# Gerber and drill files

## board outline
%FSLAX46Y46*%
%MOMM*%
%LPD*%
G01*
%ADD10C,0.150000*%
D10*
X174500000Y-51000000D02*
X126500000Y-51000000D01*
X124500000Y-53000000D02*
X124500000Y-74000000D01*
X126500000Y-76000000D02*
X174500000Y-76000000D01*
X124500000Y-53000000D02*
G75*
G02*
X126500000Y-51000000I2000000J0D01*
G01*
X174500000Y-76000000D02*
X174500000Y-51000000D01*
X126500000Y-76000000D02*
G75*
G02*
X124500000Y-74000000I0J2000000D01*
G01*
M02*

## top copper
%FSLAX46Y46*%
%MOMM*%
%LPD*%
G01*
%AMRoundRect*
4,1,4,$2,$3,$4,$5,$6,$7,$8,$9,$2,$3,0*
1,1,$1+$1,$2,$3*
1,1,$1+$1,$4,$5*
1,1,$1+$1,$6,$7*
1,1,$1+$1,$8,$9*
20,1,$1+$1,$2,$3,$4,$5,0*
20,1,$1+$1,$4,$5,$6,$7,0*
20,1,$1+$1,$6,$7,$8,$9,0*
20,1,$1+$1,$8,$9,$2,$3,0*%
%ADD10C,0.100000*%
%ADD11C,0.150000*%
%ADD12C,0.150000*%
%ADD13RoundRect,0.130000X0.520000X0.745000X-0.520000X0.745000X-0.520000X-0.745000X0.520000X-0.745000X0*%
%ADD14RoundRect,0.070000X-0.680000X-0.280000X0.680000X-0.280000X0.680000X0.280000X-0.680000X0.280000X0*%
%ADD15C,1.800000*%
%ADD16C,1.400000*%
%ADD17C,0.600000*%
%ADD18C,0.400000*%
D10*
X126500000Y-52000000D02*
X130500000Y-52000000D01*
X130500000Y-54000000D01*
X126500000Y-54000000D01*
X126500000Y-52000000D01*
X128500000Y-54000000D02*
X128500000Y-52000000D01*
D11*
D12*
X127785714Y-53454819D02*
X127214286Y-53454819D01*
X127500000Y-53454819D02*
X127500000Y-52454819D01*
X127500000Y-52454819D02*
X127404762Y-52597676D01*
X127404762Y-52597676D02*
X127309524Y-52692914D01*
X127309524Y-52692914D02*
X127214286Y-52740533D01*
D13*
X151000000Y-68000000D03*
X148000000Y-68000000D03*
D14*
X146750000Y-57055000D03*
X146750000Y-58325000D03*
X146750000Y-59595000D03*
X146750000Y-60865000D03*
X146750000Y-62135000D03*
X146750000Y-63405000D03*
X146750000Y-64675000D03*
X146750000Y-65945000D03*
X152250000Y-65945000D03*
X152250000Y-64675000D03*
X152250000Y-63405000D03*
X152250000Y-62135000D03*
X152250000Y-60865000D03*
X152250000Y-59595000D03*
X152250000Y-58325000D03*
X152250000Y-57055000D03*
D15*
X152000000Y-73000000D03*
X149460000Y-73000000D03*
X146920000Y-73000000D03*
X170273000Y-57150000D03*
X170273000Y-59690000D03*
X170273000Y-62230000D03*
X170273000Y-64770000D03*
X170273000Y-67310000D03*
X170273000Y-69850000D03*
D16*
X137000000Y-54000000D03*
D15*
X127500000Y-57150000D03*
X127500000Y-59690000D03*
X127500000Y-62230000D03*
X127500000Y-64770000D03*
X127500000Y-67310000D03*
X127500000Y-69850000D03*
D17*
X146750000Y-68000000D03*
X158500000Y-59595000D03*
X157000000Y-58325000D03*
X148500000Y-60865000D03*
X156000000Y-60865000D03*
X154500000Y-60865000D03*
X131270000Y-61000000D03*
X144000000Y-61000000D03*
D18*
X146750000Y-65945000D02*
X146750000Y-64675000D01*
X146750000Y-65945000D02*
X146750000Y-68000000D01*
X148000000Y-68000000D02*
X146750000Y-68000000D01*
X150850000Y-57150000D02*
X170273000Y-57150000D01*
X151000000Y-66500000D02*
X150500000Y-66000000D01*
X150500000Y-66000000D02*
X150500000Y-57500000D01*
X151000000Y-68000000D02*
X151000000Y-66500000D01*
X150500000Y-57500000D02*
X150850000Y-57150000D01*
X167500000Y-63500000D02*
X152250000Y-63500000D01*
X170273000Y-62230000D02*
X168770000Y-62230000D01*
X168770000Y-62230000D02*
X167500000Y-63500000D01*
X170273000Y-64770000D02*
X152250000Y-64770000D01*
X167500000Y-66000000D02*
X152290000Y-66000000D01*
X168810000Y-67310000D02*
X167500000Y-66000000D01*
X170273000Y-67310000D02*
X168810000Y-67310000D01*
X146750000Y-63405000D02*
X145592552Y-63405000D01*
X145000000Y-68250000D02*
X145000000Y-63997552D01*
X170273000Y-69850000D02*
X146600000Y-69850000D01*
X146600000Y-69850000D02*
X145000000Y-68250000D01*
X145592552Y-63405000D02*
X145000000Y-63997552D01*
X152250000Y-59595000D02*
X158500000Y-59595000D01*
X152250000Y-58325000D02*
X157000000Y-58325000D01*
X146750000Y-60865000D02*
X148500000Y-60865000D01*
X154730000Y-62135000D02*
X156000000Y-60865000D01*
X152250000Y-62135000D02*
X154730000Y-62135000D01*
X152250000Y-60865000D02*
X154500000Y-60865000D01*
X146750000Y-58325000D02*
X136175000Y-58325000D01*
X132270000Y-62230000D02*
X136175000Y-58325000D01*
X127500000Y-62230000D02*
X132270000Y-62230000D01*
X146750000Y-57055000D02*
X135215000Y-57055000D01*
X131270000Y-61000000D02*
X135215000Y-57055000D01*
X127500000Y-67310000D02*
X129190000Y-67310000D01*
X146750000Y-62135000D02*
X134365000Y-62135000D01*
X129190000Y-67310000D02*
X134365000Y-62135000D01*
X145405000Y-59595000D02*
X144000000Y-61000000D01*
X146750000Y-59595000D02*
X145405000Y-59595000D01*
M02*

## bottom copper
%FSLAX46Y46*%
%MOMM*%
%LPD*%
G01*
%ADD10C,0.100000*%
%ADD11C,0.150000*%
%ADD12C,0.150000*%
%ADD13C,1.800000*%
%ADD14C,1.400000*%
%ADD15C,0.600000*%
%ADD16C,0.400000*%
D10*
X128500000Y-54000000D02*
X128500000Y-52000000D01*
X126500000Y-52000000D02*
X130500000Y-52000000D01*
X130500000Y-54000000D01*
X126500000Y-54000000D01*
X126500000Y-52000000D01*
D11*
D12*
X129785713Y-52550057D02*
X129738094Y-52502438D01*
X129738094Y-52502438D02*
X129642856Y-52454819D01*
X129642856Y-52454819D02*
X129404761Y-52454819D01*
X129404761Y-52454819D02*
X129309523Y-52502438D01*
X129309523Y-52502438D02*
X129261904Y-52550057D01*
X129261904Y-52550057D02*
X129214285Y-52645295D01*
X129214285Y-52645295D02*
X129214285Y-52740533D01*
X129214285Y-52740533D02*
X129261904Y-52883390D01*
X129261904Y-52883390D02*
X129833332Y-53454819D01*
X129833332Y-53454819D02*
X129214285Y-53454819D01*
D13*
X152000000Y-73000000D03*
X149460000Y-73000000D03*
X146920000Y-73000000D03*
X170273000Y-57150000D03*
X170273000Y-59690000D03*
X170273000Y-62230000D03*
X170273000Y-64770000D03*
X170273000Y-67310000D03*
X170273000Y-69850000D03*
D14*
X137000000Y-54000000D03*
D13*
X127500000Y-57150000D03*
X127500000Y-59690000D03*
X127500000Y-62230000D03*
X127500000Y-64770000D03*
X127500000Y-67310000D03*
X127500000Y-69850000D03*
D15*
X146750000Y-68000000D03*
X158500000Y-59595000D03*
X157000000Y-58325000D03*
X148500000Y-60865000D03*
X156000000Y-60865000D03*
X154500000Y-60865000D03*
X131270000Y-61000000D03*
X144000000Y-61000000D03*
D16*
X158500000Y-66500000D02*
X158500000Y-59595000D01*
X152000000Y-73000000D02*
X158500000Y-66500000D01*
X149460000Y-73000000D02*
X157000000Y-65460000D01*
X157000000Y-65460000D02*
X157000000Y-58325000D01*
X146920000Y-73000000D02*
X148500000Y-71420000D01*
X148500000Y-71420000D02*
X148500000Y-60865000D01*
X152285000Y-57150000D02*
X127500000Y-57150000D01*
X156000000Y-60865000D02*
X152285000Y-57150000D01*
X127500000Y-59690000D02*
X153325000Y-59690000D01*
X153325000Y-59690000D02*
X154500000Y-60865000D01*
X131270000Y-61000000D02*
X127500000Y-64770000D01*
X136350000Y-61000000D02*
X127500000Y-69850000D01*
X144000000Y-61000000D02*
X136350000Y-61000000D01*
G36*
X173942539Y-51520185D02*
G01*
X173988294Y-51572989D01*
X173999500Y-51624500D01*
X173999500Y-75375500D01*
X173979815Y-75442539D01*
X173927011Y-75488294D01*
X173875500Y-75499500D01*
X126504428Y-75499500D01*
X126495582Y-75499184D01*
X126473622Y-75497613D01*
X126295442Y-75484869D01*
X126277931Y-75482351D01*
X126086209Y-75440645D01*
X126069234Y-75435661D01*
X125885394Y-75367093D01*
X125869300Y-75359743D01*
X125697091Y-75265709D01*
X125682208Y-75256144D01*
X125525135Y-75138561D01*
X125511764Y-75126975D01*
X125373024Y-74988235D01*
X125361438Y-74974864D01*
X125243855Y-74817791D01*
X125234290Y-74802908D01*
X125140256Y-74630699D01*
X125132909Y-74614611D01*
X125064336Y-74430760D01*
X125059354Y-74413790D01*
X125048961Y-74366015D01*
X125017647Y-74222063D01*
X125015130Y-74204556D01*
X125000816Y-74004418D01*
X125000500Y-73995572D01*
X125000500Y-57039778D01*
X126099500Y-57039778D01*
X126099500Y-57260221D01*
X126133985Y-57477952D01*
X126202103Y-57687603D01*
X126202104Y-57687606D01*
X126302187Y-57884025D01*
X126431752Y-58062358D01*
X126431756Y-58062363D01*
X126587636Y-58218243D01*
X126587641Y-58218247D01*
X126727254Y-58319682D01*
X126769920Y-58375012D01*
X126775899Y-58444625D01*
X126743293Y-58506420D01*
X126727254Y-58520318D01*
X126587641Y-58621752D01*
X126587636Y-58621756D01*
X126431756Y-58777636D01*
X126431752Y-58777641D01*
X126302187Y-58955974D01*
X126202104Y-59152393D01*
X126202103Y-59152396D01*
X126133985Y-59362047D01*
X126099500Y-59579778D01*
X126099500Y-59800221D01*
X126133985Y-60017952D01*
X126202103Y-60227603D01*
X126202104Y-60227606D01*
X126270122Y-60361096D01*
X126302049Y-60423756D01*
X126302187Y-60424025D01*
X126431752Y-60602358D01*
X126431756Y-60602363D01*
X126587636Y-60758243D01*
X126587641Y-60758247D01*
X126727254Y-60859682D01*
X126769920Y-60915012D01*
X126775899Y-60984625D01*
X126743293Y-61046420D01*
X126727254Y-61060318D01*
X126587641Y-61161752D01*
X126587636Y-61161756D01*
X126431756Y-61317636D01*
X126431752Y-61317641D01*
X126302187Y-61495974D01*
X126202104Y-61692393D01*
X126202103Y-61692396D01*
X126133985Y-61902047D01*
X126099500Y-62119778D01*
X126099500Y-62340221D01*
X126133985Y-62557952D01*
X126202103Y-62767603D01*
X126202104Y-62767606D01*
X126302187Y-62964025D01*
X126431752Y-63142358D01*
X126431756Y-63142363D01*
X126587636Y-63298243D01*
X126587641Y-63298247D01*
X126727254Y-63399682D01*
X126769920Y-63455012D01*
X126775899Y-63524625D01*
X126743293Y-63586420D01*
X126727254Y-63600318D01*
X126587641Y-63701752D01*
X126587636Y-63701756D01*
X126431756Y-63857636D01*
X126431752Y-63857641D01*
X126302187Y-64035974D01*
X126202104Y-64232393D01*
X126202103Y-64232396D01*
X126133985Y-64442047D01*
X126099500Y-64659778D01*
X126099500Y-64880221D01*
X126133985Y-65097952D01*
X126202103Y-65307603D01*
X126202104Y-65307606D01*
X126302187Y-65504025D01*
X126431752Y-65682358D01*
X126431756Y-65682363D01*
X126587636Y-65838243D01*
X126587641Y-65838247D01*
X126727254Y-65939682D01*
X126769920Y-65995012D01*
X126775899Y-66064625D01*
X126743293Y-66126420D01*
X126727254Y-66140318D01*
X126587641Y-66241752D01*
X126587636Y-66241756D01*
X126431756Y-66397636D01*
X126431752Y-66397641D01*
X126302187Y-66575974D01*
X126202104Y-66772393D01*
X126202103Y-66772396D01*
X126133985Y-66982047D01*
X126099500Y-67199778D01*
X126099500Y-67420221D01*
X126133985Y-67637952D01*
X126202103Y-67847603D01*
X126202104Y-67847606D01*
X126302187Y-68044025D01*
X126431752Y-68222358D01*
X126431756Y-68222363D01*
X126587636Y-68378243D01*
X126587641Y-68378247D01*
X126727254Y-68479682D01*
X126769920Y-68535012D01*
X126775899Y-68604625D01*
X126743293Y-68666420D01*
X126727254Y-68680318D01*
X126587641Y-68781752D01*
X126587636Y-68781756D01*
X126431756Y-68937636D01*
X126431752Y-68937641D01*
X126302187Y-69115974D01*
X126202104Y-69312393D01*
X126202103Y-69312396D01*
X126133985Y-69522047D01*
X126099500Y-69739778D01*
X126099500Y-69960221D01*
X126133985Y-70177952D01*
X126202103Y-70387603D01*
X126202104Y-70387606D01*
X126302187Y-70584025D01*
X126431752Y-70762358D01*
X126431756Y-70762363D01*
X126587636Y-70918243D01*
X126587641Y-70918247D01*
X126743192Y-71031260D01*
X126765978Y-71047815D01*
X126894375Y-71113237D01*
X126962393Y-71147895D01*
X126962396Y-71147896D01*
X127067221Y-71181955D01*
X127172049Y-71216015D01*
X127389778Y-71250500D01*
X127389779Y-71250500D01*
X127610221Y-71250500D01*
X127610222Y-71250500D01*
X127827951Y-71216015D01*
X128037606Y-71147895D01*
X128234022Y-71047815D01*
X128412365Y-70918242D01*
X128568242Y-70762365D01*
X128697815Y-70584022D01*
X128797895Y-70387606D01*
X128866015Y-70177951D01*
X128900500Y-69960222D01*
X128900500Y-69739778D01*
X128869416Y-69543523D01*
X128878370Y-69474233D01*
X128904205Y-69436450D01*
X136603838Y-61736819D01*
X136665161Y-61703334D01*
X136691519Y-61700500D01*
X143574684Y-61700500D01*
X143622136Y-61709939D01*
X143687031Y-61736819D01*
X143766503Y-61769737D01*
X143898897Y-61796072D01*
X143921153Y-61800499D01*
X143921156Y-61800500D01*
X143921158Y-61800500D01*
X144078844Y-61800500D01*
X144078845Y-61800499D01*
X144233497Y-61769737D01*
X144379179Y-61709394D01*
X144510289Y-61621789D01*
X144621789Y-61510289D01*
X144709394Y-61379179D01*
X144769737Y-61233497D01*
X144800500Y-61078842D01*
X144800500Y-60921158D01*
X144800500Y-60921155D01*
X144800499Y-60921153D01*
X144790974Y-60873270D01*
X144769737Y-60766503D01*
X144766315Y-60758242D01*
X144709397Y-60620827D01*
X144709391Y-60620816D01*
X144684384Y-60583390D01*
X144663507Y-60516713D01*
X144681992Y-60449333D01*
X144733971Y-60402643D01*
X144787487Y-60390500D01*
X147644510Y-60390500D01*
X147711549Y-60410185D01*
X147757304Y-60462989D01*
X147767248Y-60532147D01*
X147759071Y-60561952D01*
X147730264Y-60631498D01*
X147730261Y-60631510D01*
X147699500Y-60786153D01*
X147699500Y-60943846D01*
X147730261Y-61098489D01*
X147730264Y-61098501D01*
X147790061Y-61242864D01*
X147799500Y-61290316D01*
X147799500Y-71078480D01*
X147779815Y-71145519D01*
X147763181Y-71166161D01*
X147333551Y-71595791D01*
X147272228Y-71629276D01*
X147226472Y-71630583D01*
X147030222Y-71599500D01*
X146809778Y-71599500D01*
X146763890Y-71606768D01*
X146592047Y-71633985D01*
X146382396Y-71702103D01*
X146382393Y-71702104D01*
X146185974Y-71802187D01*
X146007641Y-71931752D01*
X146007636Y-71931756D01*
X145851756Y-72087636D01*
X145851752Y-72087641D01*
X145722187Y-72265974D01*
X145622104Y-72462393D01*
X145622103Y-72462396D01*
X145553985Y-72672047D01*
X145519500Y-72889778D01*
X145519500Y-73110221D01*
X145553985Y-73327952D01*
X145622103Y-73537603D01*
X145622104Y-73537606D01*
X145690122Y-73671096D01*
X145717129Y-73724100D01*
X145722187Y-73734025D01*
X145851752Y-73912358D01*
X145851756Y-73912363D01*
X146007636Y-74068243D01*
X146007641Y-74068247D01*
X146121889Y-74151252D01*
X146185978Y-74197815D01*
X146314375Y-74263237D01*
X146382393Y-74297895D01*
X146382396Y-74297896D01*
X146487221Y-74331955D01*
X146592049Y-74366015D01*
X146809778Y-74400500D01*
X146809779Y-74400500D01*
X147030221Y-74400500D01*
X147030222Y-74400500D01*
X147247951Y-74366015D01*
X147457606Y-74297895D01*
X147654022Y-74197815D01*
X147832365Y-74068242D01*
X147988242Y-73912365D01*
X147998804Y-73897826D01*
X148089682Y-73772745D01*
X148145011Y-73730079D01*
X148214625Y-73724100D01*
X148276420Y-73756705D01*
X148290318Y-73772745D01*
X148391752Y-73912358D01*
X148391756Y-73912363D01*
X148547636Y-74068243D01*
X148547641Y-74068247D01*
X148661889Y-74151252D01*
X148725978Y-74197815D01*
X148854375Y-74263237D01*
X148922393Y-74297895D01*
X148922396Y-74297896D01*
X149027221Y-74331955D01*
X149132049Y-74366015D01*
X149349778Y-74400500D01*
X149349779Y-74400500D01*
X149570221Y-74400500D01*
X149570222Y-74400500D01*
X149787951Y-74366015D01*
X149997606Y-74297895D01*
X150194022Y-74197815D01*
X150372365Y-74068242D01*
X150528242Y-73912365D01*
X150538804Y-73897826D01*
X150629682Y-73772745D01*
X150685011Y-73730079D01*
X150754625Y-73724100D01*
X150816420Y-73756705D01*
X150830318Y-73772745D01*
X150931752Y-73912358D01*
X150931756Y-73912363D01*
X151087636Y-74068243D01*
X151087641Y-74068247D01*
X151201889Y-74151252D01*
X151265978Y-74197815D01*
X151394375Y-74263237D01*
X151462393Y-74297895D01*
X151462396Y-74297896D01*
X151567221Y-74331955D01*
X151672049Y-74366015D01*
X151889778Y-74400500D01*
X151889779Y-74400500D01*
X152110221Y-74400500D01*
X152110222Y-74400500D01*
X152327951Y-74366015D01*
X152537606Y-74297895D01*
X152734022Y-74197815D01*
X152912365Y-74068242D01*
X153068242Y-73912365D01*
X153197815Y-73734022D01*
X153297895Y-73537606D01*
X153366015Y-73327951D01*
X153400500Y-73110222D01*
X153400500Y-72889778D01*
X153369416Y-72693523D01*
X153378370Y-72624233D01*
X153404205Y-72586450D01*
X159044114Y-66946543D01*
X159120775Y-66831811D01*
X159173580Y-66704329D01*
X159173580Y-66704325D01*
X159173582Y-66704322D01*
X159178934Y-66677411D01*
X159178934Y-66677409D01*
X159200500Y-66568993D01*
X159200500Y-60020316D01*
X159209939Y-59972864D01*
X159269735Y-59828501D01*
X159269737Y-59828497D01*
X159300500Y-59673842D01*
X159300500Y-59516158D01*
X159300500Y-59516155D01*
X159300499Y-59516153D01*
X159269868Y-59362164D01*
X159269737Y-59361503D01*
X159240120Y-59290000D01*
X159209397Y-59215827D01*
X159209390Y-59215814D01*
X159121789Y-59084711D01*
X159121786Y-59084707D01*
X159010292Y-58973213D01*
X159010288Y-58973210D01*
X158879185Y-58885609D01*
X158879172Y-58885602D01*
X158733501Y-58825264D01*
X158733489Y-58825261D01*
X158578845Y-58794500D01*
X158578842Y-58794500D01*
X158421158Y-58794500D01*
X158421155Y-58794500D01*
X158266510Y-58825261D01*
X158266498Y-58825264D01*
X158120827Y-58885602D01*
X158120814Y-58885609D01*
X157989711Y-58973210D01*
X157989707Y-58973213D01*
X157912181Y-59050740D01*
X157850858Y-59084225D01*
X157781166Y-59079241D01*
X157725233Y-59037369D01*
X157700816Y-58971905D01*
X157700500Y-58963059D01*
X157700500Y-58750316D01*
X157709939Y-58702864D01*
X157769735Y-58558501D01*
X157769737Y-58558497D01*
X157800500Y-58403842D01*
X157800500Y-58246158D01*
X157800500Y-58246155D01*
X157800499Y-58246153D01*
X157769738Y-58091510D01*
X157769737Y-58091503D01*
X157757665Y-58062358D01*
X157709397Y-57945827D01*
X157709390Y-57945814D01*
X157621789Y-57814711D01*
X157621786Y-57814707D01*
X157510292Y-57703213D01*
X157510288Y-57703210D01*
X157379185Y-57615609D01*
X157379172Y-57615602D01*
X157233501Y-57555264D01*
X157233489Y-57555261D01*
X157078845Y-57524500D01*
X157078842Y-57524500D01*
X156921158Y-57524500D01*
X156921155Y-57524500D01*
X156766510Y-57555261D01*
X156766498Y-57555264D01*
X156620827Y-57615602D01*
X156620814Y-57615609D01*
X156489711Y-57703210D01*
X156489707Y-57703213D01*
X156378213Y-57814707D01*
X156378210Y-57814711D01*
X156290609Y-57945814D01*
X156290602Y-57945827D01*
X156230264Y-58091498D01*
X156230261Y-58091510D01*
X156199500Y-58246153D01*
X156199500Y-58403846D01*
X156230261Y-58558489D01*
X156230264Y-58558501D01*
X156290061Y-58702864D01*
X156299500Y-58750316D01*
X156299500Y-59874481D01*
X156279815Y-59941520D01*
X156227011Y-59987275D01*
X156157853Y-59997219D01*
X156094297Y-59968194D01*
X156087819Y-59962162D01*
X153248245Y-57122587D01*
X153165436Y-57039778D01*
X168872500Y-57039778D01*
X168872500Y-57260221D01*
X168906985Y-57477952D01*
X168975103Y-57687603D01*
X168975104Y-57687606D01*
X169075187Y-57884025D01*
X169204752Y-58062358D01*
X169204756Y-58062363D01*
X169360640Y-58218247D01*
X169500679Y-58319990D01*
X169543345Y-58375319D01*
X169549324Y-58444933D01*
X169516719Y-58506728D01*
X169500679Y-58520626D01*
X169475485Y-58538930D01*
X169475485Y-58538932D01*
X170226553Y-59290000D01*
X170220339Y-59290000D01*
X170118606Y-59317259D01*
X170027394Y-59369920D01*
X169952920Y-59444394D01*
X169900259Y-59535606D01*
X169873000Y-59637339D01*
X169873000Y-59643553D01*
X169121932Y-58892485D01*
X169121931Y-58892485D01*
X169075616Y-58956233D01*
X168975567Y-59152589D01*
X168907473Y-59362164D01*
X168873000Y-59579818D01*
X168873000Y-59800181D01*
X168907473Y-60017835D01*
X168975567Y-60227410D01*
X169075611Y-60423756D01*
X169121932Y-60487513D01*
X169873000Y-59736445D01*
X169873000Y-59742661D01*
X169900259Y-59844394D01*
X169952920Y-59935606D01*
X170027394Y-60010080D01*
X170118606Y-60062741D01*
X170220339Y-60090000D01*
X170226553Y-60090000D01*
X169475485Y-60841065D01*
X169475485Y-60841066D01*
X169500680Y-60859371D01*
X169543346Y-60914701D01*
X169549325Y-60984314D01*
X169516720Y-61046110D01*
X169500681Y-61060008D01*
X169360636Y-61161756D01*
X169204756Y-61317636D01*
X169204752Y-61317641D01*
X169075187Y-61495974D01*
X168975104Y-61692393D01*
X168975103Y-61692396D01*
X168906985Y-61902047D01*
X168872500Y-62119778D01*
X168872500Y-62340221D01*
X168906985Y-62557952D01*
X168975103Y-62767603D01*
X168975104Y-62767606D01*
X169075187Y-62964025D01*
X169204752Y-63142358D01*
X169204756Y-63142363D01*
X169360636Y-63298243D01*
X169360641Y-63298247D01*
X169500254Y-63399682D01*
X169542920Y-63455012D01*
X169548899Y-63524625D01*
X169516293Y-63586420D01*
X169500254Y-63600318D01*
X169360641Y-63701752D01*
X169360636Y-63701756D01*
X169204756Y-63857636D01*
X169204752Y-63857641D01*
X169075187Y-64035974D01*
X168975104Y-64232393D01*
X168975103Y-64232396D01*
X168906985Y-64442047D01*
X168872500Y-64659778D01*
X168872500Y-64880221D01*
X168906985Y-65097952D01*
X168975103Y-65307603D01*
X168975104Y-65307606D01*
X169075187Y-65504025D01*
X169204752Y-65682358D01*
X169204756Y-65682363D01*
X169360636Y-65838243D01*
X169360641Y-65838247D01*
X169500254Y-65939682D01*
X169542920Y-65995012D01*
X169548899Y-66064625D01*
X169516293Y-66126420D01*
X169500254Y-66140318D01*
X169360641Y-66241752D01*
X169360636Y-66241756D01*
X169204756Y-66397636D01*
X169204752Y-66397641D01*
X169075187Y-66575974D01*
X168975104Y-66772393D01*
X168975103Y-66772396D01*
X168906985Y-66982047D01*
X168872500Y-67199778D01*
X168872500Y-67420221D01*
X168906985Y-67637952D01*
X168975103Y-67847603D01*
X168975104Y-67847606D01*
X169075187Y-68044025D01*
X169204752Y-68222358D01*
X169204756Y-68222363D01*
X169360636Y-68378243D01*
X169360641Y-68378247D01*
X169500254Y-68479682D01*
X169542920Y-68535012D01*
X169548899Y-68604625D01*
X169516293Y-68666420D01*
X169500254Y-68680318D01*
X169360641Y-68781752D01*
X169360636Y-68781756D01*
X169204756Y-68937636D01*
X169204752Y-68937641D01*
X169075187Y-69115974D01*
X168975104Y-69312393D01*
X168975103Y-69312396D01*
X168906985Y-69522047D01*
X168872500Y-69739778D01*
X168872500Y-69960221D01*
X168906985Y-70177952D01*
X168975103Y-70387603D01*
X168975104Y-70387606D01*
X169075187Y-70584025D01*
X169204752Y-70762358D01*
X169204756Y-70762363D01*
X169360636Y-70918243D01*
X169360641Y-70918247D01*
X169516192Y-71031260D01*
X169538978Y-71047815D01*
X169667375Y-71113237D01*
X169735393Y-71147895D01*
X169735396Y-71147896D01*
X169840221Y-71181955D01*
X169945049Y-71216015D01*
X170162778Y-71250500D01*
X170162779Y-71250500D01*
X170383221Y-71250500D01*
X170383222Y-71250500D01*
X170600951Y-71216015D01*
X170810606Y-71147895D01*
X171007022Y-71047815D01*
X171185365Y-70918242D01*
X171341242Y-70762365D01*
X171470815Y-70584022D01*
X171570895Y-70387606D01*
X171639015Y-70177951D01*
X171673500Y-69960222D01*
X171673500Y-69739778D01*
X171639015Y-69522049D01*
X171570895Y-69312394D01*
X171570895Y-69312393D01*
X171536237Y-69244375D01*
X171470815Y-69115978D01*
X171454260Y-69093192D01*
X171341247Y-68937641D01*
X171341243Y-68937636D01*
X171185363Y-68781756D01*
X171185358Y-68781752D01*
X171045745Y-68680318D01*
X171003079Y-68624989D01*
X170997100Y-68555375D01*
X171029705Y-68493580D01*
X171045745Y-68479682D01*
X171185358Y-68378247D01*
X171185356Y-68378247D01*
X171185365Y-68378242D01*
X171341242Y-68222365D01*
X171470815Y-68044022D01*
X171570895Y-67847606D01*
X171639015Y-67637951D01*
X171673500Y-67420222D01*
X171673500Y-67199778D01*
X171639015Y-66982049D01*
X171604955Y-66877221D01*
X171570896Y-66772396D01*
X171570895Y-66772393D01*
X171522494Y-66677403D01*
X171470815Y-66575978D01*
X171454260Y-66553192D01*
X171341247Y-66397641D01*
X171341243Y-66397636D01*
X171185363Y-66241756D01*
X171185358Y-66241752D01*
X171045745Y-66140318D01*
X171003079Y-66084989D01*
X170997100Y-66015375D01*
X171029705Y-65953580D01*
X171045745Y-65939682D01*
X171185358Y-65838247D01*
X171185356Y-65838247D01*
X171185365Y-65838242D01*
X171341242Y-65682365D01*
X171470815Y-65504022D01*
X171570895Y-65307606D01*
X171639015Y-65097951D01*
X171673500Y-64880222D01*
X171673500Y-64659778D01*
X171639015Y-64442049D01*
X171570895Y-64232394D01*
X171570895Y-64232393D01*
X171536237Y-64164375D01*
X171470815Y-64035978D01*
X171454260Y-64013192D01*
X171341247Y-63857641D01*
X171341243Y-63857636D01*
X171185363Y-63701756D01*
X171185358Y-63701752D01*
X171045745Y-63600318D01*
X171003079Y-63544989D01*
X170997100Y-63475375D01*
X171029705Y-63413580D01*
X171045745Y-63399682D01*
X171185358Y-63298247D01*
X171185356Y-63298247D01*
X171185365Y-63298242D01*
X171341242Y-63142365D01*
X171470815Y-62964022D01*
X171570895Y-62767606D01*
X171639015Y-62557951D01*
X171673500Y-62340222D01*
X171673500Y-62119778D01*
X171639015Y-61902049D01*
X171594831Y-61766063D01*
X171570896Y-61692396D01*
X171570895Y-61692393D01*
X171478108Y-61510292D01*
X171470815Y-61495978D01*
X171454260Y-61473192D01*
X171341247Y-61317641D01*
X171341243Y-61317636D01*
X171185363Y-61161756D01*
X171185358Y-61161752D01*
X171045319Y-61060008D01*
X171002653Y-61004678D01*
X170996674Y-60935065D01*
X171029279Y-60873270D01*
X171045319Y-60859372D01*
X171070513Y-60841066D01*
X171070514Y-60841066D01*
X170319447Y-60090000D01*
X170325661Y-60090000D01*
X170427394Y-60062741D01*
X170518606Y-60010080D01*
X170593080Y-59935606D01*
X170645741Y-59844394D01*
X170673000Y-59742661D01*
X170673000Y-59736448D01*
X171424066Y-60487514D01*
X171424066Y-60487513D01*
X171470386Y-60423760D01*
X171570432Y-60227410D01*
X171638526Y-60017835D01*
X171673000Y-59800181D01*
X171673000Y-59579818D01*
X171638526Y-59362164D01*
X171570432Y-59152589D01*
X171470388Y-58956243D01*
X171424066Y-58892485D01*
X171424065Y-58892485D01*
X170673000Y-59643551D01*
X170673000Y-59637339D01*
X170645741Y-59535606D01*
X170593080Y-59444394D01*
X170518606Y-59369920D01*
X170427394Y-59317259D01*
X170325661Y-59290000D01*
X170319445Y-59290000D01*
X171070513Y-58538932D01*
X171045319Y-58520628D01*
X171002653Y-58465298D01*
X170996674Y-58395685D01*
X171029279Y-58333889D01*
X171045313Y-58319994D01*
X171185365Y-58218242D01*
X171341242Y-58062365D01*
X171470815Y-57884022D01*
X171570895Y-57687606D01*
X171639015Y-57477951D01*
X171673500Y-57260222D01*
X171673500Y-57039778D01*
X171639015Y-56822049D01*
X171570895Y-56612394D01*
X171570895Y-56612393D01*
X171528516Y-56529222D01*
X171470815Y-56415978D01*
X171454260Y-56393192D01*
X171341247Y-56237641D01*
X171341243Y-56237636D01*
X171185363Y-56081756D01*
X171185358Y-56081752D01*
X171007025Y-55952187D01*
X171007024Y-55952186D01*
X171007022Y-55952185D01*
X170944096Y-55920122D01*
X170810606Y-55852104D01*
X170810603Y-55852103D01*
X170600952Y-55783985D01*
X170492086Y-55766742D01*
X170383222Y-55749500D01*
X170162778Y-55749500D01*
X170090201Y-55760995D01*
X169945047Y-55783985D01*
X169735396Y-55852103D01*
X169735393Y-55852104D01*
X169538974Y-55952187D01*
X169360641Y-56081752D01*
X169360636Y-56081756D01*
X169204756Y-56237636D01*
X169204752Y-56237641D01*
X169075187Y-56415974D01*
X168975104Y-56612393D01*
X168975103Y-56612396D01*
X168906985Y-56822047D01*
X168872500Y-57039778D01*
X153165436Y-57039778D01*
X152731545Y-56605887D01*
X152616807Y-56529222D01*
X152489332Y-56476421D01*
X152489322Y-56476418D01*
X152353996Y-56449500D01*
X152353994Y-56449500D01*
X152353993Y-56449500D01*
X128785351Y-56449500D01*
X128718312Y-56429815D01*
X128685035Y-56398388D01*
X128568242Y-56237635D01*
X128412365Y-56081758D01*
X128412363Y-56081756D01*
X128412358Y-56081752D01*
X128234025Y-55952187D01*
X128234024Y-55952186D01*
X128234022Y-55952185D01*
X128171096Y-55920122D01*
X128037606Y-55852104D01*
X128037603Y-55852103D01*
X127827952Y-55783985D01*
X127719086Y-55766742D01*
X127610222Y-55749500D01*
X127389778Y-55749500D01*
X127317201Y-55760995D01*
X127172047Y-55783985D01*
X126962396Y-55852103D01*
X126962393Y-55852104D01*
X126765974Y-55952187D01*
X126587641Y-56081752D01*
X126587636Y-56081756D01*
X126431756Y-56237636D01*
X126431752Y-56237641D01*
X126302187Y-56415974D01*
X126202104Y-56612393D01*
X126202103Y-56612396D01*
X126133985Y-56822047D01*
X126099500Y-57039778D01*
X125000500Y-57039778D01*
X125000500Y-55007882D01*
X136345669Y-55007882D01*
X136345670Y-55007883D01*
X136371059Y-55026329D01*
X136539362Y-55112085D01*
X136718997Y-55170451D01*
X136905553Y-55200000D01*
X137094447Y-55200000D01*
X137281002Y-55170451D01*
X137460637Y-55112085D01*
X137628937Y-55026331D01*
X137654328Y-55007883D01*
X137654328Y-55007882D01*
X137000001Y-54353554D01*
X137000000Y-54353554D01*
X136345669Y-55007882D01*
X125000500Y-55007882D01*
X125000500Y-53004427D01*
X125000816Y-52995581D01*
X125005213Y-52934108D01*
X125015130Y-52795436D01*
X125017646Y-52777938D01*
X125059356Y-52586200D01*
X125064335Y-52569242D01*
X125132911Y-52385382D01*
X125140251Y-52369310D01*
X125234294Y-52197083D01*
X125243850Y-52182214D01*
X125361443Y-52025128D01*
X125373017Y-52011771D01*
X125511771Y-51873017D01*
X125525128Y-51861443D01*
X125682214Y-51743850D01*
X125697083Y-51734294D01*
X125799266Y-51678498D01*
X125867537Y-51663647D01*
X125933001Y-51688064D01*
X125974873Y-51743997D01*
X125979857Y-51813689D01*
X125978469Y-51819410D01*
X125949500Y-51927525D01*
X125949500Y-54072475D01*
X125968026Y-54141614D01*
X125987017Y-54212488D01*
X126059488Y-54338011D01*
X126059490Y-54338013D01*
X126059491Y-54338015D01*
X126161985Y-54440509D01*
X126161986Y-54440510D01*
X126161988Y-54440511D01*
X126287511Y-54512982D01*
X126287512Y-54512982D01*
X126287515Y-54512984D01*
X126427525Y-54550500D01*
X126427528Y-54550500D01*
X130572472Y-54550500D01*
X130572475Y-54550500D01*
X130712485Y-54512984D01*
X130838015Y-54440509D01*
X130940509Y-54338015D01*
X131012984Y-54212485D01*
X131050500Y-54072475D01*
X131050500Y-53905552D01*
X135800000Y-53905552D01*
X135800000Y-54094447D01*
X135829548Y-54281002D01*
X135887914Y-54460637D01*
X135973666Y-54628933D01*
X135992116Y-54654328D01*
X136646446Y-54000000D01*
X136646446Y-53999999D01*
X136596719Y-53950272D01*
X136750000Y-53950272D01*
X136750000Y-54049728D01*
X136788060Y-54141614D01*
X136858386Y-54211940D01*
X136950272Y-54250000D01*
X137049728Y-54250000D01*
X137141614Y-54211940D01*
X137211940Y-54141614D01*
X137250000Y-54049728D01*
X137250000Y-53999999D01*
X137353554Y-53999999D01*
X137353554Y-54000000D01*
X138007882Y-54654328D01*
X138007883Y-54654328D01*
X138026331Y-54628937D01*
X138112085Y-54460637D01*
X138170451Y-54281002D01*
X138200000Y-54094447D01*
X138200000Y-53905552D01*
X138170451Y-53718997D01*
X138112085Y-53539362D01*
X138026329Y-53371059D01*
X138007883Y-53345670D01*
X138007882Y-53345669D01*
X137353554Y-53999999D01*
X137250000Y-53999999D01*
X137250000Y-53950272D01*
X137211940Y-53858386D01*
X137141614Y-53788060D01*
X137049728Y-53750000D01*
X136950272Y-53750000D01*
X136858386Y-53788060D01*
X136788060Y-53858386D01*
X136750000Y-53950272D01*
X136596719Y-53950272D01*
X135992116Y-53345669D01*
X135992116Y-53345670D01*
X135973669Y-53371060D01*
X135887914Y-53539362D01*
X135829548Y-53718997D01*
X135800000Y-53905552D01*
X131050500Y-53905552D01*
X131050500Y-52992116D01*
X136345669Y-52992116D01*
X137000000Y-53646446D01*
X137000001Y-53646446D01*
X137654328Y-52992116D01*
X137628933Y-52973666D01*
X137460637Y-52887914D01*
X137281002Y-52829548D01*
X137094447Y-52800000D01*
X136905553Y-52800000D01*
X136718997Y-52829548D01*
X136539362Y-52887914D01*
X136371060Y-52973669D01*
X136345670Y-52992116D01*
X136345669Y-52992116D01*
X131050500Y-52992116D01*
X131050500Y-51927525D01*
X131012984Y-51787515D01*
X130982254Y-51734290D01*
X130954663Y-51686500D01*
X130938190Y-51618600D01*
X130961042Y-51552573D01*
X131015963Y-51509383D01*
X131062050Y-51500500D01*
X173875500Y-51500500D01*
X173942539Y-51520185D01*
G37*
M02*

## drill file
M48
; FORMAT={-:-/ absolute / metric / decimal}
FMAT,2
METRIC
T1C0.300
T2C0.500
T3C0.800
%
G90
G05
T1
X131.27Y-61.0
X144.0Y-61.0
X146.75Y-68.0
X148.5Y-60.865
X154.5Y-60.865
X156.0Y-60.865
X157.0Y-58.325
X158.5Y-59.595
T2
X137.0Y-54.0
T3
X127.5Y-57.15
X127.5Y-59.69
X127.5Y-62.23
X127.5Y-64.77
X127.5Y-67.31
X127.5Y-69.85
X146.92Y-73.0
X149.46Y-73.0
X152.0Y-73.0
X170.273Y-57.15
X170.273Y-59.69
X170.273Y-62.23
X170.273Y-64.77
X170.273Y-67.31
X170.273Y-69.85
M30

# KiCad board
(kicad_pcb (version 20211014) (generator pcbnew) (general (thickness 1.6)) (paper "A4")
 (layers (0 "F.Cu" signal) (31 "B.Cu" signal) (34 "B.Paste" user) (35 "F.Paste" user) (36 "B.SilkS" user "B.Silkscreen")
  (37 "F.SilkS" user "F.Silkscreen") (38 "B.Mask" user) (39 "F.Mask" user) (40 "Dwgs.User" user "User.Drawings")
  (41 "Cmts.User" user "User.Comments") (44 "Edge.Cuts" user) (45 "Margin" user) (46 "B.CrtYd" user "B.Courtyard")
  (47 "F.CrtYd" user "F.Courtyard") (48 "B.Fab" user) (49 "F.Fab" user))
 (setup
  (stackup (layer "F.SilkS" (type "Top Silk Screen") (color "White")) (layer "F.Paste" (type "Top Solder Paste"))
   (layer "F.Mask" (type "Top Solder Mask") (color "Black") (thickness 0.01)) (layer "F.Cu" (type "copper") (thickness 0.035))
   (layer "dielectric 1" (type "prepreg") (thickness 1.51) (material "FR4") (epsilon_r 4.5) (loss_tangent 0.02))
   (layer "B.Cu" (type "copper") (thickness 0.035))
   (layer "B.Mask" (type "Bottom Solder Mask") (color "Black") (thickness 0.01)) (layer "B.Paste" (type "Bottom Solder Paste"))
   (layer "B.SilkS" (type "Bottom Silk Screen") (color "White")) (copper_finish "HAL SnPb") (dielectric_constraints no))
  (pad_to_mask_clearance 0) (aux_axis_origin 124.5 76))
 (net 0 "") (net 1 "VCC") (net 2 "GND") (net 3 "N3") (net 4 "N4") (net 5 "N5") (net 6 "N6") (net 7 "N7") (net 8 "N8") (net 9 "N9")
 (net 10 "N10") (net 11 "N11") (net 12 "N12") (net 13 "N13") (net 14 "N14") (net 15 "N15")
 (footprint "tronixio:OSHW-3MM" (layer "F.Cu") (at 172.5 73.5)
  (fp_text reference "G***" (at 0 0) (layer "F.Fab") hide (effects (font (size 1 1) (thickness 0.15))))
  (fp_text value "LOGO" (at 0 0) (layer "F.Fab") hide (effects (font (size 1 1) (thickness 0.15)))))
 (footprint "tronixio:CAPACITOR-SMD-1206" (layer "F.Cu") (at 149.5 68 180) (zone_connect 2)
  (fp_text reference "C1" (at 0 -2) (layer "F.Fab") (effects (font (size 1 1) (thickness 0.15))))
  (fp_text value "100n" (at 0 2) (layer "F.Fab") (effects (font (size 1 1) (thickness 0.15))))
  (pad "1" smd roundrect (at -1.5 0 180) (size 1.3 1.75) (layers "F.Cu" "F.Paste" "F.Mask") (roundrect_rratio 0.1) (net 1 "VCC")
   (zone_connect 2))
  (pad "2" smd roundrect (at 1.5 0 180) (size 1.3 1.75) (layers "F.Cu" "F.Paste" "F.Mask") (roundrect_rratio 0.1) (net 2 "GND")
   (zone_connect 2)))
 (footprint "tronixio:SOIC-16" (layer "F.Cu") (at 149.5 61.5)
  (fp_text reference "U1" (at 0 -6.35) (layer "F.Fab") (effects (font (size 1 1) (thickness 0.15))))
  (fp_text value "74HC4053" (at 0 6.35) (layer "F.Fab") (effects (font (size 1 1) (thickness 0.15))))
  (pad "1" smd roundrect (at -2.75 -4.445) (size 1.5 0.7) (layers "F.Cu" "F.Paste" "F.Mask") (roundrect_rratio 0.1) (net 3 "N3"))
  (pad "2" smd roundrect (at -2.75 -3.175) (size 1.5 0.7) (layers "F.Cu" "F.Paste" "F.Mask") (roundrect_rratio 0.1) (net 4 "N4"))
  (pad "3" smd roundrect (at -2.75 -1.905) (size 1.5 0.7) (layers "F.Cu" "F.Paste" "F.Mask") (roundrect_rratio 0.1) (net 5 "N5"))
  (pad "4" smd roundrect (at -2.75 -0.635) (size 1.5 0.7) (layers "F.Cu" "F.Paste" "F.Mask") (roundrect_rratio 0.1) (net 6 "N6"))
  (pad "5" smd roundrect (at -2.75 0.635) (size 1.5 0.7) (layers "F.Cu" "F.Paste" "F.Mask") (roundrect_rratio 0.1) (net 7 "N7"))
  (pad "6" smd roundrect (at -2.75 1.905) (size 1.5 0.7) (layers "F.Cu" "F.Paste" "F.Mask") (roundrect_rratio 0.1) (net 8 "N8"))
  (pad "7" smd roundrect (at -2.75 3.175) (size 1.5 0.7) (layers "F.Cu" "F.Paste" "F.Mask") (roundrect_rratio 0.1) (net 2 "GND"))
  (pad "8" smd roundrect (at -2.75 4.445) (size 1.5 0.7) (layers "F.Cu" "F.Paste" "F.Mask") (roundrect_rratio 0.1) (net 2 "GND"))
  (pad "9" smd roundrect (at 2.75 4.445) (size 1.5 0.7) (layers "F.Cu" "F.Paste" "F.Mask") (roundrect_rratio 0.1) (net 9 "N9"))
  (pad "10" smd roundrect (at 2.75 3.175) (size 1.5 0.7) (layers "F.Cu" "F.Paste" "F.Mask") (roundrect_rratio 0.1) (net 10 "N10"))
  (pad "11" smd roundrect (at 2.75 1.905) (size 1.5 0.7) (layers "F.Cu" "F.Paste" "F.Mask") (roundrect_rratio 0.1) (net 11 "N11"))
  (pad "12" smd roundrect (at 2.75 0.635) (size 1.5 0.7) (layers "F.Cu" "F.Paste" "F.Mask") (roundrect_rratio 0.1) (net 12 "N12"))
  (pad "13" smd roundrect (at 2.75 -0.635) (size 1.5 0.7) (layers "F.Cu" "F.Paste" "F.Mask") (roundrect_rratio 0.1) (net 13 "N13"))
  (pad "14" smd roundrect (at 2.75 -1.905) (size 1.5 0.7) (layers "F.Cu" "F.Paste" "F.Mask") (roundrect_rratio 0.1) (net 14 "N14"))
  (pad "15" smd roundrect (at 2.75 -3.175) (size 1.5 0.7) (layers "F.Cu" "F.Paste" "F.Mask") (roundrect_rratio 0.1) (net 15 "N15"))
  (pad "16" smd roundrect (at 2.75 -4.445) (size 1.5 0.7) (layers "F.Cu" "F.Paste" "F.Mask") (roundrect_rratio 0.1) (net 1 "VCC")))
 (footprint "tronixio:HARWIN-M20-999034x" (layer "F.Cu") (at 152 73 -90)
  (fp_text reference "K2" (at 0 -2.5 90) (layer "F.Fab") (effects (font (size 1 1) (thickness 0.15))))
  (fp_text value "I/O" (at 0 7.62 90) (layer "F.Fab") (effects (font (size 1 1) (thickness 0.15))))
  (pad "1" thru_hole circle locked (at 0 0 270) (size 1.8 1.8) (drill 0.8) (layers *.Cu *.Mask) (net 14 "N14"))
  (pad "2" thru_hole circle (at 0 2.54 270) (size 1.8 1.8) (drill 0.8) (layers *.Cu *.Mask) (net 15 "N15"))
  (pad "3" thru_hole circle (at 0 5.08 270) (size 1.8 1.8) (drill 0.8) (layers *.Cu *.Mask) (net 6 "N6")))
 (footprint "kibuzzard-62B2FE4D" (layer "F.Cu") (at 166.75 59.69)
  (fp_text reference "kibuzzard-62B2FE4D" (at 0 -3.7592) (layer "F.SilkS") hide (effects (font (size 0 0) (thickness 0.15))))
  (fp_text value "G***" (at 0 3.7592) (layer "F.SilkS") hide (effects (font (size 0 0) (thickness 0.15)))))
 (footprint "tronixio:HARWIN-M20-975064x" (layer "F.Cu") (at 170.273 57.15 -90)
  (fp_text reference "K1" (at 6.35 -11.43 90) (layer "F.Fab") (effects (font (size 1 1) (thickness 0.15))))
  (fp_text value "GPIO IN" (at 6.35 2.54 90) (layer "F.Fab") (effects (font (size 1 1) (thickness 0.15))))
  (pad "1" thru_hole circle (at 0 0 270) (size 1.8 1.8) (drill 0.8) (layers *.Cu *.Mask) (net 1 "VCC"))
  (pad "2" thru_hole circle (at 2.54 0 270) (size 1.8 1.8) (drill 0.8) (layers *.Cu *.Mask) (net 2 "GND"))
  (pad "3" thru_hole circle (at 5.08 0 270) (size 1.8 1.8) (drill 0.8) (layers *.Cu *.Mask) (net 11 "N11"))
  (pad "4" thru_hole circle (at 7.62 0 270) (size 1.8 1.8) (drill 0.8) (layers *.Cu *.Mask) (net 10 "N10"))
  (pad "5" thru_hole circle (at 10.16 0 270) (size 1.8 1.8) (drill 0.8) (layers *.Cu *.Mask) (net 9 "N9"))
  (pad "6" thru_hole circle (at 12.7 0 270) (size 1.8 1.8) (drill 0.8) (layers *.Cu *.Mask) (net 8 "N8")))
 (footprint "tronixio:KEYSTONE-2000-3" (layer "F.Cu") (at 137 54)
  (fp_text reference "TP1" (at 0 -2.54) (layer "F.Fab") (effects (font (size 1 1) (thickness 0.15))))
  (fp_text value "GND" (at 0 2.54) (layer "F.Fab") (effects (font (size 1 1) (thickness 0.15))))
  (pad "1" thru_hole circle (at 0 0) (size 1.4 1.4) (drill 0.5) (layers *.Cu *.Mask) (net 2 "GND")))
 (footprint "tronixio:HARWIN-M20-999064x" (layer "F.Cu") (at 127.5 57.15)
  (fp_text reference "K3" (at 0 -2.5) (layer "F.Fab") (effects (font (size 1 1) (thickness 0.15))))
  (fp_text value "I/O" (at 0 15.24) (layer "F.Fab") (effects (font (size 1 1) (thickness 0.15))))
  (pad "1" thru_hole circle locked (at 0 0) (size 1.8 1.8) (drill 0.8) (layers *.Cu *.Mask) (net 12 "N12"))
  (pad "2" thru_hole circle (at 0 2.54) (size 1.8 1.8) (drill 0.8) (layers *.Cu *.Mask) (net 13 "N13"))
  (pad "3" thru_hole circle (at 0 5.08) (size 1.8 1.8) (drill 0.8) (layers *.Cu *.Mask) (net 4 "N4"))
  (pad "4" thru_hole circle (at 0 7.62) (size 1.8 1.8) (drill 0.8) (layers *.Cu *.Mask) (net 3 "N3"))
  (pad "5" thru_hole circle (at 0 10.16) (size 1.8 1.8) (drill 0.8) (layers *.Cu *.Mask) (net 7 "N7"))
  (pad "6" thru_hole circle (at 0 12.7) (size 1.8 1.8) (drill 0.8) (layers *.Cu *.Mask) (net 5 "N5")))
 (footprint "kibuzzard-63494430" (layer "F.Cu") (at 140.5 54)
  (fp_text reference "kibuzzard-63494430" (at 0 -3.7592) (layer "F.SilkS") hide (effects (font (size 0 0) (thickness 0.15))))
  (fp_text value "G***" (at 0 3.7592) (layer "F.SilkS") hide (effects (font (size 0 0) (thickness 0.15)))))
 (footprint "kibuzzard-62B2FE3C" (layer "F.Cu") (at 166.75 57.15)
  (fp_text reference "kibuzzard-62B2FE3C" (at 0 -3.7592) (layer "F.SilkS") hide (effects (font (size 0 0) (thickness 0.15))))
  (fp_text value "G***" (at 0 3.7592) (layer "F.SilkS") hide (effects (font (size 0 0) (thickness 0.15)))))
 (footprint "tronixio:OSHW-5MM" (layer "B.Cu") (at 149.5 57 180)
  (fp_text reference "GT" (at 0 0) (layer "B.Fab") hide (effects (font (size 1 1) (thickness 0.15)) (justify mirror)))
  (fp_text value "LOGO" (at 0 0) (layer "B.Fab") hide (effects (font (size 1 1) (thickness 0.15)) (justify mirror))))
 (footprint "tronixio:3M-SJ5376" (layer "B.Cu") (at 134.5 63.5 180)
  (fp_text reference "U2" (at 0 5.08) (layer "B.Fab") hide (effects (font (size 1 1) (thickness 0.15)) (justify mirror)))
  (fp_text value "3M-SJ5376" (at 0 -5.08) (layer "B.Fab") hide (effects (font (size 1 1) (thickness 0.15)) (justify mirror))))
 (gr_rect (start 126.5 54) (end 130.5 52) (layer "F.Cu") (width 0.1) (fill none))
 (gr_line (start 128.5 54) (end 128.5 52) (layer "F.Cu") (width 0.1))
 (gr_line (start 128.5 54) (end 128.5 52) (layer "B.Cu") (width 0.1))
 (gr_rect (start 126.5 54) (end 130.5 52) (layer "B.Cu") (width 0.1) (fill none))
 (gr_line (start 174.5 51) (end 126.5 51) (layer "Edge.Cuts") (width 0.15))
 (gr_line (start 124.5 53) (end 124.5 74) (layer "Edge.Cuts") (width 0.15))
 (gr_line (start 126.5 76) (end 174.5 76) (layer "Edge.Cuts") (width 0.15))
 (gr_arc (start 124.5 53) (mid 125.085786 51.585786) (end 126.5 51) (layer "Edge.Cuts") (width 0.15))
 (gr_line (start 174.5 76) (end 174.5 51) (layer "Edge.Cuts") (width 0.15))
 (gr_arc (start 126.5 76) (mid 125.085786 75.414214) (end 124.5 74) (layer "Edge.Cuts") (width 0.15))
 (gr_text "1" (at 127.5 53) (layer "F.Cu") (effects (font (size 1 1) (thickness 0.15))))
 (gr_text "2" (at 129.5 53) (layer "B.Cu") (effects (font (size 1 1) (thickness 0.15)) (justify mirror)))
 (segment (start 146.75 65.945) (end 146.75 64.675) (width 0.4) (layer "F.Cu") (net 2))
 (segment (start 146.75 65.945) (end 146.75 68) (width 0.4) (layer "F.Cu") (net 2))
 (segment (start 148 68) (end 146.75 68) (width 0.4) (layer "F.Cu") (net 2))
 (via (at 146.75 68) (size 0.6) (drill 0.3) (layers "F.Cu" "B.Cu") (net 2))
 (segment (start 150.85 57.15) (end 170.273 57.15) (width 0.4) (layer "F.Cu") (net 1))
 (segment (start 151 66.5) (end 150.5 66) (width 0.4) (layer "F.Cu") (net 1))
 (segment (start 150.5 66) (end 150.5 57.5) (width 0.4) (layer "F.Cu") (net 1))
 (segment (start 151 68) (end 151 66.5) (width 0.4) (layer "F.Cu") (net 1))
 (segment (start 150.5 57.5) (end 150.85 57.15) (width 0.4) (layer "F.Cu") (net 1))
 (segment (start 167.5 63.5) (end 152.25 63.5) (width 0.4) (layer "F.Cu") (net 11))
 (segment (start 170.273 62.23) (end 168.77 62.23) (width 0.4) (layer "F.Cu") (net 11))
 (segment (start 168.77 62.23) (end 167.5 63.5) (width 0.4) (layer "F.Cu") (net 11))
 (segment (start 170.273 64.77) (end 152.25 64.77) (width 0.4) (layer "F.Cu") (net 10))
 (segment (start 167.5 66) (end 152.29 66) (width 0.4) (layer "F.Cu") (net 9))
 (segment (start 168.81 67.31) (end 167.5 66) (width 0.4) (layer "F.Cu") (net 9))
 (segment (start 170.273 67.31) (end 168.81 67.31) (width 0.4) (layer "F.Cu") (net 9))
 (segment (start 146.75 63.405) (end 145.592552 63.405) (width 0.4) (layer "F.Cu") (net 8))
 (segment (start 145 68.25) (end 145 63.997552) (width 0.4) (layer "F.Cu") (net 8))
 (segment (start 170.273 69.85) (end 146.6 69.85) (width 0.4) (layer "F.Cu") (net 8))
 (segment (start 146.6 69.85) (end 145 68.25) (width 0.4) (layer "F.Cu") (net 8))
 (segment (start 145.592552 63.405) (end 145 63.997552) (width 0.4) (layer "F.Cu") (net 8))
 (segment (start 152.25 59.595) (end 158.5 59.595) (width 0.4) (layer "F.Cu") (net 14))
 (via (at 158.5 59.595) (size 0.6) (drill 0.3) (layers "F.Cu" "B.Cu") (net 14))
 (segment (start 158.5 66.5) (end 158.5 59.595) (width 0.4) (layer "B.Cu") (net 14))
 (segment (start 152 73) (end 158.5 66.5) (width 0.4) (layer "B.Cu") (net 14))
 (segment (start 152.25 58.325) (end 157 58.325) (width 0.4) (layer "F.Cu") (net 15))
 (via (at 157 58.325) (size 0.6) (drill 0.3) (layers "F.Cu" "B.Cu") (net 15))
 (segment (start 149.46 73) (end 157 65.46) (width 0.4) (layer "B.Cu") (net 15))
 (segment (start 157 65.46) (end 157 58.325) (width 0.4) (layer "B.Cu") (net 15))
 (segment (start 146.75 60.865) (end 148.5 60.865) (width 0.4) (layer "F.Cu") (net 6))
 (via (at 148.5 60.865) (size 0.6) (drill 0.3) (layers "F.Cu" "B.Cu") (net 6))
 (segment (start 146.92 73) (end 148.5 71.42) (width 0.4) (layer "B.Cu") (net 6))
 (segment (start 148.5 71.42) (end 148.5 60.865) (width 0.4) (layer "B.Cu") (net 6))
 (segment (start 154.73 62.135) (end 156 60.865) (width 0.4) (layer "F.Cu") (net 12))
 (segment (start 152.25 62.135) (end 154.73 62.135) (width 0.4) (layer "F.Cu") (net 12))
 (via (at 156 60.865) (size 0.6) (drill 0.3) (layers "F.Cu" "B.Cu") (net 12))
 (segment (start 152.285 57.15) (end 127.5 57.15) (width 0.4) (layer "B.Cu") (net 12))
 (segment (start 156 60.865) (end 152.285 57.15) (width 0.4) (layer "B.Cu") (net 12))
 (segment (start 152.25 60.865) (end 154.5 60.865) (width 0.4) (layer "F.Cu") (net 13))
 (via (at 154.5 60.865) (size 0.6) (drill 0.3) (layers "F.Cu" "B.Cu") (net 13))
 (segment (start 127.5 59.69) (end 153.325 59.69) (width 0.4) (layer "B.Cu") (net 13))
 (segment (start 153.325 59.69) (end 154.5 60.865) (width 0.4) (layer "B.Cu") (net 13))
 (segment (start 146.75 58.325) (end 136.175 58.325) (width 0.4) (layer "F.Cu") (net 4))
 (segment (start 132.27 62.23) (end 136.175 58.325) (width 0.4) (layer "F.Cu") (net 4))
 (segment (start 127.5 62.23) (end 132.27 62.23) (width 0.4) (layer "F.Cu") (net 4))
 (segment (start 146.75 57.055) (end 135.215 57.055) (width 0.4) (layer "F.Cu") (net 3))
 (segment (start 131.27 61) (end 135.215 57.055) (width 0.4) (layer "F.Cu") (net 3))
 (via (at 131.27 61) (size 0.6) (drill 0.3) (layers "F.Cu" "B.Cu") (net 3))
 (segment (start 131.27 61) (end 127.5 64.77) (width 0.4) (layer "B.Cu") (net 3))
 (segment (start 127.5 67.31) (end 129.19 67.31) (width 0.4) (layer "F.Cu") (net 7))
 (segment (start 146.75 62.135) (end 134.365 62.135) (width 0.4) (layer "F.Cu") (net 7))
 (segment (start 129.19 67.31) (end 134.365 62.135) (width 0.4) (layer "F.Cu") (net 7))
 (segment (start 145.405 59.595) (end 144 61) (width 0.4) (layer "F.Cu") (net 5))
 (segment (start 146.75 59.595) (end 145.405 59.595) (width 0.4) (layer "F.Cu") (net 5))
 (via (at 144 61) (size 0.6) (drill 0.3) (layers "F.Cu" "B.Cu") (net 5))
 (segment (start 136.35 61) (end 127.5 69.85) (width 0.4) (layer "B.Cu") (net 5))
 (segment (start 144 61) (end 136.35 61) (width 0.4) (layer "B.Cu") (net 5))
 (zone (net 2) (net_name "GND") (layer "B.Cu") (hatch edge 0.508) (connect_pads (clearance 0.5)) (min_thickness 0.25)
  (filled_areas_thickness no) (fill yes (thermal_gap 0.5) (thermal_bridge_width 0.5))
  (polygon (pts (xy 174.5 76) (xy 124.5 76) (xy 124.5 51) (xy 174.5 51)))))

